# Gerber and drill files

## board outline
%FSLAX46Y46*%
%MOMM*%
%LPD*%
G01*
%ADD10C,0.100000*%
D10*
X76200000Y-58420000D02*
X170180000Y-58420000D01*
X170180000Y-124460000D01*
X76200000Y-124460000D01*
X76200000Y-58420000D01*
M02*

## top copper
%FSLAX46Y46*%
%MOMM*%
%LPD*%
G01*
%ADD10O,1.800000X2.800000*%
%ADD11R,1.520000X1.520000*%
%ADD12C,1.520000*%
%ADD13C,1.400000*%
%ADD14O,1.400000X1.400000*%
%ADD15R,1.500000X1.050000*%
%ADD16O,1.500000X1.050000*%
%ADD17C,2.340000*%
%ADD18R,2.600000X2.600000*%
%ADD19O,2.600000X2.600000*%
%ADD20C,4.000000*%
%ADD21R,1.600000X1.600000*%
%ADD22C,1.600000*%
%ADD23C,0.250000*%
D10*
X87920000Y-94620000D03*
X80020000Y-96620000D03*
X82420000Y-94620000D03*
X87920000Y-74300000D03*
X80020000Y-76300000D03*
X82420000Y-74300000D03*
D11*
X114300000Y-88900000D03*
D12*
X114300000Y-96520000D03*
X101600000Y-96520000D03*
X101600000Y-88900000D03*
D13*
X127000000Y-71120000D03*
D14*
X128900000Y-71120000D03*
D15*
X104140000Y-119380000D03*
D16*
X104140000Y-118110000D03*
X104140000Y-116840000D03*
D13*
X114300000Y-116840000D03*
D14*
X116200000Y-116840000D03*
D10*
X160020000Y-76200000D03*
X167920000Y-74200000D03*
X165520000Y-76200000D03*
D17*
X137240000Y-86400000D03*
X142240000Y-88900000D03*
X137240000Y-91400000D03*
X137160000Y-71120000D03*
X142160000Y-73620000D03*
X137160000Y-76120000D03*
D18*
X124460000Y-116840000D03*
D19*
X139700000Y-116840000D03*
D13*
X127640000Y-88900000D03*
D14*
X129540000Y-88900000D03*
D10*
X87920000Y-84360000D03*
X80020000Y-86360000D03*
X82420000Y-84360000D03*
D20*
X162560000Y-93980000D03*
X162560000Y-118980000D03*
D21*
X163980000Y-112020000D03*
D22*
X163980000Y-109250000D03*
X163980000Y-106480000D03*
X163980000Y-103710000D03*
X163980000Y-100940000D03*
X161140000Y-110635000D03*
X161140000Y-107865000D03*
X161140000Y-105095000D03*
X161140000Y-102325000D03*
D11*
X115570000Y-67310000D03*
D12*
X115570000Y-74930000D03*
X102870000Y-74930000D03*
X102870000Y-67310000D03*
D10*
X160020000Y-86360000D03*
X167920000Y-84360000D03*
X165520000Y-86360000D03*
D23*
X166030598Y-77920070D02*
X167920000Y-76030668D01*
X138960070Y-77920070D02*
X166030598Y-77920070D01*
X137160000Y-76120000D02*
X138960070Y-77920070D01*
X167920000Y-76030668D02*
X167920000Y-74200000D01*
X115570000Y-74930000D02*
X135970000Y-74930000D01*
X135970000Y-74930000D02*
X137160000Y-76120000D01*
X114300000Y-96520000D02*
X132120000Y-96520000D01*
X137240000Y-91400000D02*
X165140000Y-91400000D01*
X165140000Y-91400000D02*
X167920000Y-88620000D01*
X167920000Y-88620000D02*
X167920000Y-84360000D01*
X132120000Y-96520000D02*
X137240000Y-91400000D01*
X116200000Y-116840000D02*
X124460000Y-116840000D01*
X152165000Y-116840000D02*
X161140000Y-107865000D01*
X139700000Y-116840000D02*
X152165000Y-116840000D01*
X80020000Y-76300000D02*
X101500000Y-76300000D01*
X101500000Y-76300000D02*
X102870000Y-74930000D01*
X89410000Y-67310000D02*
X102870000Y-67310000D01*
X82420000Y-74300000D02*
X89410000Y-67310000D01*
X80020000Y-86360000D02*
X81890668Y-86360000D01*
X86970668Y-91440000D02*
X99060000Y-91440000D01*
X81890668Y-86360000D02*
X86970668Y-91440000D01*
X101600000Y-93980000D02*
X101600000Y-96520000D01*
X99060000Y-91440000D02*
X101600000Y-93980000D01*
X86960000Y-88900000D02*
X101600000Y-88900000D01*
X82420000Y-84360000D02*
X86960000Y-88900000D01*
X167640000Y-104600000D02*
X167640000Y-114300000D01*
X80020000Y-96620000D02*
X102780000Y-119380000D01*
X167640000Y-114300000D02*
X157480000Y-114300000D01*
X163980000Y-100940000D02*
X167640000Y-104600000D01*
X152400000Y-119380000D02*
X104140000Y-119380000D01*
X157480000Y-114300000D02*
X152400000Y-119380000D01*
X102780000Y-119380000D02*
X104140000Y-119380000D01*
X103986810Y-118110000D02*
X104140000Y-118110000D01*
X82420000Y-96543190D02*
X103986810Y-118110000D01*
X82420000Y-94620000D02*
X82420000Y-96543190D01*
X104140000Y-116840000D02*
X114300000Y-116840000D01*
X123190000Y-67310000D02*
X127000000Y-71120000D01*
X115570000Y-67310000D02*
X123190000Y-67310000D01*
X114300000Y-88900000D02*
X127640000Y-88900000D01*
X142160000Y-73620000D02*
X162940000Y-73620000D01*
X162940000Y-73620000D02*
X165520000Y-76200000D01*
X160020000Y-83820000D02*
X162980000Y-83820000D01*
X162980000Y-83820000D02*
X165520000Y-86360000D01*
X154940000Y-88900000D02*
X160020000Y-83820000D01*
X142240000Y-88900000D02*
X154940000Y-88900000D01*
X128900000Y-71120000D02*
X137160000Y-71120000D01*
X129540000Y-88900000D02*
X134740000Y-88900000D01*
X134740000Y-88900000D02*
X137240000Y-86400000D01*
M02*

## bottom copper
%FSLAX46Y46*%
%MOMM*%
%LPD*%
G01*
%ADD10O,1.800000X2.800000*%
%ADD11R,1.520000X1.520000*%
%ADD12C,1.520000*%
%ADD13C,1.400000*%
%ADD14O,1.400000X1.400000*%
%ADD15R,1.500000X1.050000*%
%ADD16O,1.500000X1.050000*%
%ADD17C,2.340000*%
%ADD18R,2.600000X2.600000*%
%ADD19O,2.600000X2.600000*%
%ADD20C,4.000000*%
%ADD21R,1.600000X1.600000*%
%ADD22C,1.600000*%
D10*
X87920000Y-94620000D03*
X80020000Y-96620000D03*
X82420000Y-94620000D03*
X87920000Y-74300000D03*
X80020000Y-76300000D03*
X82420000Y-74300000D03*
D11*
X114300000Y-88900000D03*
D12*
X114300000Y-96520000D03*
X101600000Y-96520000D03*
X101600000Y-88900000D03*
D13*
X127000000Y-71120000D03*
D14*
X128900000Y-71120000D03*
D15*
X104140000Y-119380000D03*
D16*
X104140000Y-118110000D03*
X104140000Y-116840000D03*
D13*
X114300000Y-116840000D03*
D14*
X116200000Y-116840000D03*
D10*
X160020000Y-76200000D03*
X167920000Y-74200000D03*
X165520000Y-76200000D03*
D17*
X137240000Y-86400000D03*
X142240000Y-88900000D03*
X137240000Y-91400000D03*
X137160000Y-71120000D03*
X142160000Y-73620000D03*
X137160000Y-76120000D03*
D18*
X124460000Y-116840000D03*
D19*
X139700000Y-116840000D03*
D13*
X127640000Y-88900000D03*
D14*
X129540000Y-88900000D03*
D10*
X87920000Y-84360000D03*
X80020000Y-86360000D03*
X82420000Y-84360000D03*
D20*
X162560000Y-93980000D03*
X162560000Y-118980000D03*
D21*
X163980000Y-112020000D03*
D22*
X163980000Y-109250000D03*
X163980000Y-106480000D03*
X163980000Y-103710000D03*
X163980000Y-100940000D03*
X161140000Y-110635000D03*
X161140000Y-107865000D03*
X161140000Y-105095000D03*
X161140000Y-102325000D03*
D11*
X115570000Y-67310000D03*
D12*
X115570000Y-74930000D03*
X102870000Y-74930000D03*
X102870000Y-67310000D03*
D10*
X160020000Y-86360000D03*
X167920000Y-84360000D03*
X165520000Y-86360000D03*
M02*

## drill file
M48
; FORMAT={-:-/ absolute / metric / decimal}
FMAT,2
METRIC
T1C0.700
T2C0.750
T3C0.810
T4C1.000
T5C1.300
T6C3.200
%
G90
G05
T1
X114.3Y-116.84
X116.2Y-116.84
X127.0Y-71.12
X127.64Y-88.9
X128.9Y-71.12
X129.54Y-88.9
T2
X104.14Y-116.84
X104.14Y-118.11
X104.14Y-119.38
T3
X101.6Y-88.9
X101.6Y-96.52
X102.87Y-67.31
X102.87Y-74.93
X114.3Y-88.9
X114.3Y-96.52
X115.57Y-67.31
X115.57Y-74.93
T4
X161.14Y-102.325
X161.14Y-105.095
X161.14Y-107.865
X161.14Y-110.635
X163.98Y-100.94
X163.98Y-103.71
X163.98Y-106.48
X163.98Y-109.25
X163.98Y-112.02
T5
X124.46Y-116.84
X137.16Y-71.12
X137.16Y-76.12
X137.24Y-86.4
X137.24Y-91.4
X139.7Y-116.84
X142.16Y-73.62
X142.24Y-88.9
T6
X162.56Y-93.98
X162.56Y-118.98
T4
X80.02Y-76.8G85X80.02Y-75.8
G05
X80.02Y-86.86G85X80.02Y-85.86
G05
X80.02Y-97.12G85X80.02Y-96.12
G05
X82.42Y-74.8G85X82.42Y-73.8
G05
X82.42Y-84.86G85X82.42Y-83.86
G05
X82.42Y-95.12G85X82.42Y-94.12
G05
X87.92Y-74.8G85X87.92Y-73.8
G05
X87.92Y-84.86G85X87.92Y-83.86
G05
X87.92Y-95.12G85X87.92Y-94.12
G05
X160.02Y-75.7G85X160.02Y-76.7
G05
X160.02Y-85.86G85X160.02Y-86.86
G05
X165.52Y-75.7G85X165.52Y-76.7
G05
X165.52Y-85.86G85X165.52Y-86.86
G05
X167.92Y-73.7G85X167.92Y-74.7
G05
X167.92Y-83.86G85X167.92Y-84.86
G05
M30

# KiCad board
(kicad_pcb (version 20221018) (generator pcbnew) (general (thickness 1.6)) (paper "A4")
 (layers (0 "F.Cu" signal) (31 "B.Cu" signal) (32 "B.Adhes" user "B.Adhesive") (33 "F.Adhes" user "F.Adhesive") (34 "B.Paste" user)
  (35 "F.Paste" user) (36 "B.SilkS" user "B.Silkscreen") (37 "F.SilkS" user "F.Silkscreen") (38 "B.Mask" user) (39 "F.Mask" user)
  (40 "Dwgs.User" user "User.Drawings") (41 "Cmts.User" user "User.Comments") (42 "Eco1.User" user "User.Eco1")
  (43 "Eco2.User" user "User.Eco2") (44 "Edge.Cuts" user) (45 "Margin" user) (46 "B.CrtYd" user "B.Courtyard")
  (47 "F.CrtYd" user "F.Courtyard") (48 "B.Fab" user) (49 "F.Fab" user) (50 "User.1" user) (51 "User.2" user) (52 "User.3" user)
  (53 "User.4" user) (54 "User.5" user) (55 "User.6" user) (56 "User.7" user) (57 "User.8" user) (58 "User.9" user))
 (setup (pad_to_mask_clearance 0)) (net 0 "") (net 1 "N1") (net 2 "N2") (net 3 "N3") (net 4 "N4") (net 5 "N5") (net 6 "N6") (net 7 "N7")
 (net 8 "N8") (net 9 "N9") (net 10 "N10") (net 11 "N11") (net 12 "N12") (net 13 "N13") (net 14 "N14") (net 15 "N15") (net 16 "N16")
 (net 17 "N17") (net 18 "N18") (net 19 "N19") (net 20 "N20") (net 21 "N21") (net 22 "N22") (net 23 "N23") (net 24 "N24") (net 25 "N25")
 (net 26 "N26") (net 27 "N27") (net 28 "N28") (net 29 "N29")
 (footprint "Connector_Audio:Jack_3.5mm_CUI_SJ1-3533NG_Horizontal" (layer "F.Cu") (at 80.02 96.62 90)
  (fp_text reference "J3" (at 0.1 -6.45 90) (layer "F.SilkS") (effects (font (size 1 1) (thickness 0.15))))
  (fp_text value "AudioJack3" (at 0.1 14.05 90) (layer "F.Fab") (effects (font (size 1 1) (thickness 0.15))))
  (pad "R" thru_hole oval (at 2 7.9 90) (size 2.8 1.8) (drill oval 2 1) (layers "*.Cu" "*.Mask") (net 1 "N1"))
  (pad "S" thru_hole oval (at 0 0 90) (size 2.8 1.8) (drill oval 2 1) (layers "*.Cu" "*.Mask") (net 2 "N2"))
  (pad "T" thru_hole oval (at 2 2.4 90) (size 2.8 1.8) (drill oval 2 1) (layers "*.Cu" "*.Mask") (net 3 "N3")))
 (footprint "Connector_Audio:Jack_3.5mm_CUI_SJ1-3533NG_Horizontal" (layer "F.Cu") (at 80.02 76.3 90)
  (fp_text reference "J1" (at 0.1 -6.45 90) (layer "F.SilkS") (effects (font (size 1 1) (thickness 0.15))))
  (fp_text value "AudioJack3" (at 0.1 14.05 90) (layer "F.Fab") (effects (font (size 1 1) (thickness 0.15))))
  (pad "R" thru_hole oval (at 2 7.9 90) (size 2.8 1.8) (drill oval 2 1) (layers "*.Cu" "*.Mask") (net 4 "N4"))
  (pad "S" thru_hole oval (at 0 0 90) (size 2.8 1.8) (drill oval 2 1) (layers "*.Cu" "*.Mask") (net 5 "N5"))
  (pad "T" thru_hole oval (at 2 2.4 90) (size 2.8 1.8) (drill oval 2 1) (layers "*.Cu" "*.Mask") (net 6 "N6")))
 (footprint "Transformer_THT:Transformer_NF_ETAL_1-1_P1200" (layer "F.Cu") (at 114.3 88.9)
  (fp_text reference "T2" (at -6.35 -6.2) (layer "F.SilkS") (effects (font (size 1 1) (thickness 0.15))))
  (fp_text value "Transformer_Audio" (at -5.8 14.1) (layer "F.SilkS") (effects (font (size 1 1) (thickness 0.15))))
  (pad "1" thru_hole rect (at 0 0) (size 1.52 1.52) (drill 0.81) (layers "*.Cu" "*.Mask") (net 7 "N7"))
  (pad "3" thru_hole circle (at 0 7.62) (size 1.52 1.52) (drill 0.81) (layers "*.Cu" "*.Mask") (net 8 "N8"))
  (pad "4" thru_hole circle (at -12.7 7.62) (size 1.52 1.52) (drill 0.81) (layers "*.Cu" "*.Mask") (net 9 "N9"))
  (pad "6" thru_hole circle (at -12.7 0) (size 1.52 1.52) (drill 0.81) (layers "*.Cu" "*.Mask") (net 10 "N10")))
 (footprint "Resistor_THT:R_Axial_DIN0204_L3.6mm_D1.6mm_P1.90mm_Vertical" (layer "F.Cu") (at 127 71.12)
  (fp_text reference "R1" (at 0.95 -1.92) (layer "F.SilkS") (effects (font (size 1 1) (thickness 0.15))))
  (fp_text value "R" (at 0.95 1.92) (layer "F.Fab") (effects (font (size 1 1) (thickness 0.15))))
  (pad "1" thru_hole circle (at 0 0) (size 1.4 1.4) (drill 0.7) (layers "*.Cu" "*.Mask") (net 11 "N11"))
  (pad "2" thru_hole oval (at 1.9 0) (size 1.4 1.4) (drill 0.7) (layers "*.Cu" "*.Mask") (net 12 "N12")))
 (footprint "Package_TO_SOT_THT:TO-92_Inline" (layer "F.Cu") (at 104.14 119.38 90)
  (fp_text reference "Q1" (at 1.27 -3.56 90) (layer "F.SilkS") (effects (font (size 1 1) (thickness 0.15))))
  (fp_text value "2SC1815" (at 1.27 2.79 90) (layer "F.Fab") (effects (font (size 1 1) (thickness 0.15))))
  (pad "1" thru_hole rect (at 0 0 90) (size 1.05 1.5) (drill 0.75) (layers "*.Cu" "*.Mask") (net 2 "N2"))
  (pad "2" thru_hole oval (at 1.27 0 90) (size 1.05 1.5) (drill 0.75) (layers "*.Cu" "*.Mask") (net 3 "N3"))
  (pad "3" thru_hole oval (at 2.54 0 90) (size 1.05 1.5) (drill 0.75) (layers "*.Cu" "*.Mask") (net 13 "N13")))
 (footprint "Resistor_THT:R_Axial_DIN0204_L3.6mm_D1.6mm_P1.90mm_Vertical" (layer "F.Cu") (at 114.3 116.84)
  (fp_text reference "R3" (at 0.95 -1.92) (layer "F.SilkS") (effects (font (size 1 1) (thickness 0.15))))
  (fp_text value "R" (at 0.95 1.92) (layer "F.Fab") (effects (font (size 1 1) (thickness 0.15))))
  (pad "1" thru_hole circle (at 0 0) (size 1.4 1.4) (drill 0.7) (layers "*.Cu" "*.Mask") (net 13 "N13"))
  (pad "2" thru_hole oval (at 1.9 0) (size 1.4 1.4) (drill 0.7) (layers "*.Cu" "*.Mask") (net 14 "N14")))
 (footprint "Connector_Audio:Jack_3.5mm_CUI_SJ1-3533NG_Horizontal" (layer "F.Cu") (at 167.92 74.2 -90)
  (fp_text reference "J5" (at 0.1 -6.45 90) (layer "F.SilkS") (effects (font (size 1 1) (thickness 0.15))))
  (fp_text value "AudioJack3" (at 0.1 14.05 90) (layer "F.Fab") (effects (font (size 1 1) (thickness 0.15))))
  (pad "R" thru_hole oval (at 2 7.9 270) (size 2.8 1.8) (drill oval 2 1) (layers "*.Cu" "*.Mask") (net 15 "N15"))
  (pad "S" thru_hole oval (at 0 0 270) (size 2.8 1.8) (drill oval 2 1) (layers "*.Cu" "*.Mask") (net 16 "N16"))
  (pad "T" thru_hole oval (at 2 2.4 270) (size 2.8 1.8) (drill oval 2 1) (layers "*.Cu" "*.Mask") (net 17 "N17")))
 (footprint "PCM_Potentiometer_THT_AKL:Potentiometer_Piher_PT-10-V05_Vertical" (layer "F.Cu") (at 137.24 91.4)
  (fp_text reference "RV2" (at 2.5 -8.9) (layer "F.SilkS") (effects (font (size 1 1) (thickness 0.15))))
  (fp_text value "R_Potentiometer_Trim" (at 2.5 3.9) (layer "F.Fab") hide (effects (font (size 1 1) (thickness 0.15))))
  (pad "1" thru_hole circle (at 0 -5) (size 2.34 2.34) (drill 1.3) (layers "*.Cu" "*.Mask") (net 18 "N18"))
  (pad "2" thru_hole circle (at 5 -2.5) (size 2.34 2.34) (drill 1.3) (layers "*.Cu" "*.Mask") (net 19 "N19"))
  (pad "3" thru_hole circle (at 0 0) (size 2.34 2.34) (drill 1.3) (layers "*.Cu" "*.Mask") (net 8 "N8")))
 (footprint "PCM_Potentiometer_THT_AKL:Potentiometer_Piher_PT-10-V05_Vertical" (layer "F.Cu") (at 137.16 76.12)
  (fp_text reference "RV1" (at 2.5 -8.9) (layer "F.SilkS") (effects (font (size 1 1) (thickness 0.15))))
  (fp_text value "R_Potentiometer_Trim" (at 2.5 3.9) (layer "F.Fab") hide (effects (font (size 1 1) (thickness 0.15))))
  (pad "1" thru_hole circle (at 0 -5) (size 2.34 2.34) (drill 1.3) (layers "*.Cu" "*.Mask") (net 12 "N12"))
  (pad "2" thru_hole circle (at 5 -2.5) (size 2.34 2.34) (drill 1.3) (layers "*.Cu" "*.Mask") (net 17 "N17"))
  (pad "3" thru_hole circle (at 0 0) (size 2.34 2.34) (drill 1.3) (layers "*.Cu" "*.Mask") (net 16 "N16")))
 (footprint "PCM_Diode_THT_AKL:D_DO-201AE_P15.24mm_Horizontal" (layer "F.Cu") (at 124.46 116.84)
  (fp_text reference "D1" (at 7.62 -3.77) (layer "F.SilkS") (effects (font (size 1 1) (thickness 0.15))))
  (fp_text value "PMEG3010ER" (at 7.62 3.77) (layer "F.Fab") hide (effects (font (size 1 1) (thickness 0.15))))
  (pad "1" thru_hole rect (at 0 0) (size 2.6 2.6) (drill 1.3) (layers "*.Cu" "*.Mask") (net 14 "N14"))
  (pad "2" thru_hole oval (at 15.24 0) (size 2.6 2.6) (drill 1.3) (layers "*.Cu" "*.Mask") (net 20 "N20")))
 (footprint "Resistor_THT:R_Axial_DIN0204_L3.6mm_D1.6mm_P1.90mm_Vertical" (layer "F.Cu") (at 127.64 88.9)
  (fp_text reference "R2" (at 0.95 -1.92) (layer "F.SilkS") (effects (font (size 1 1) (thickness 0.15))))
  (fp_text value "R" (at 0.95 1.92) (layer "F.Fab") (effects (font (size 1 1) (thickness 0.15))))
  (pad "1" thru_hole circle (at 0 0) (size 1.4 1.4) (drill 0.7) (layers "*.Cu" "*.Mask") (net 7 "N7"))
  (pad "2" thru_hole oval (at 1.9 0) (size 1.4 1.4) (drill 0.7) (layers "*.Cu" "*.Mask") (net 18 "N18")))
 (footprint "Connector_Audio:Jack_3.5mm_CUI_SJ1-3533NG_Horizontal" (layer "F.Cu") (at 80.02 86.36 90)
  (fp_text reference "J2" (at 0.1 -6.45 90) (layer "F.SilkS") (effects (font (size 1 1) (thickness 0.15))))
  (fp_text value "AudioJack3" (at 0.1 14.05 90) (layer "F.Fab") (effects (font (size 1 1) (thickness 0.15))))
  (pad "R" thru_hole oval (at 2 7.9 90) (size 2.8 1.8) (drill oval 2 1) (layers "*.Cu" "*.Mask") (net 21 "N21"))
  (pad "S" thru_hole oval (at 0 0 90) (size 2.8 1.8) (drill oval 2 1) (layers "*.Cu" "*.Mask") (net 9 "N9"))
  (pad "T" thru_hole oval (at 2 2.4 90) (size 2.8 1.8) (drill oval 2 1) (layers "*.Cu" "*.Mask") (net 10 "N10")))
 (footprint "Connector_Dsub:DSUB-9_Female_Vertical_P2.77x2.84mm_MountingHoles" (layer "F.Cu") (at 163.98 112.02 -90)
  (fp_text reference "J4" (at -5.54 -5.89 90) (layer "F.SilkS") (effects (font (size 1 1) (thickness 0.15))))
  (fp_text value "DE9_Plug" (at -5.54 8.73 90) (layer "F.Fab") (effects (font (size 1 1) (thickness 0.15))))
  (pad "0" thru_hole circle (at -18.04 1.42 270) (size 4 4) (drill 3.2) (layers "*.Cu" "*.Mask"))
  (pad "0" thru_hole circle (at 6.96 1.42 270) (size 4 4) (drill 3.2) (layers "*.Cu" "*.Mask"))
  (pad "1" thru_hole rect (at 0 0 270) (size 1.6 1.6) (drill 1) (layers "*.Cu" "*.Mask") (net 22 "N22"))
  (pad "2" thru_hole circle (at -2.77 0 270) (size 1.6 1.6) (drill 1) (layers "*.Cu" "*.Mask") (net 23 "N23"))
  (pad "3" thru_hole circle (at -5.54 0 270) (size 1.6 1.6) (drill 1) (layers "*.Cu" "*.Mask") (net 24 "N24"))
  (pad "4" thru_hole circle (at -8.31 0 270) (size 1.6 1.6) (drill 1) (layers "*.Cu" "*.Mask") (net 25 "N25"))
  (pad "5" thru_hole circle (at -11.08 0 270) (size 1.6 1.6) (drill 1) (layers "*.Cu" "*.Mask") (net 2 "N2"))
  (pad "6" thru_hole circle (at -1.385 2.84 270) (size 1.6 1.6) (drill 1) (layers "*.Cu" "*.Mask") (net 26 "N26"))
  (pad "7" thru_hole circle (at -4.155 2.84 270) (size 1.6 1.6) (drill 1) (layers "*.Cu" "*.Mask") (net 20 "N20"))
  (pad "8" thru_hole circle (at -6.925 2.84 270) (size 1.6 1.6) (drill 1) (layers "*.Cu" "*.Mask") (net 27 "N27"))
  (pad "9" thru_hole circle (at -9.695 2.84 270) (size 1.6 1.6) (drill 1) (layers "*.Cu" "*.Mask") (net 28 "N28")))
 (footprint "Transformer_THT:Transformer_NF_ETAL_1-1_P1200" (layer "F.Cu") (at 115.57 67.31)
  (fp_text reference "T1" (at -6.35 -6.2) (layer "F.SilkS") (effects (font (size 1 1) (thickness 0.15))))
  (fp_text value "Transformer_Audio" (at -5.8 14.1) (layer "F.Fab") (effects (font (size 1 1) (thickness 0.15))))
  (pad "1" thru_hole rect (at 0 0) (size 1.52 1.52) (drill 0.81) (layers "*.Cu" "*.Mask") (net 11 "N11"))
  (pad "3" thru_hole circle (at 0 7.62) (size 1.52 1.52) (drill 0.81) (layers "*.Cu" "*.Mask") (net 16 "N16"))
  (pad "4" thru_hole circle (at -12.7 7.62) (size 1.52 1.52) (drill 0.81) (layers "*.Cu" "*.Mask") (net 5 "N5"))
  (pad "6" thru_hole circle (at -12.7 0) (size 1.52 1.52) (drill 0.81) (layers "*.Cu" "*.Mask") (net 6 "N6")))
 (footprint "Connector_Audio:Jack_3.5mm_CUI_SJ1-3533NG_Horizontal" (layer "F.Cu") (at 167.92 84.36 -90)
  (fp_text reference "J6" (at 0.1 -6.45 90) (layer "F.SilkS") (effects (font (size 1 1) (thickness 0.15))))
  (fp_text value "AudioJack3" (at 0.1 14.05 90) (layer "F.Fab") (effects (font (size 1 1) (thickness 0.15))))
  (pad "R" thru_hole oval (at 2 7.9 270) (size 2.8 1.8) (drill oval 2 1) (layers "*.Cu" "*.Mask") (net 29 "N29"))
  (pad "S" thru_hole oval (at 0 0 270) (size 2.8 1.8) (drill oval 2 1) (layers "*.Cu" "*.Mask") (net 8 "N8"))
  (pad "T" thru_hole oval (at 2 2.4 270) (size 2.8 1.8) (drill oval 2 1) (layers "*.Cu" "*.Mask") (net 19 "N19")))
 (gr_rect (start 76.2 58.42) (end 170.18 124.46) (stroke (width 0.1) (type default)) (fill none) (layer "Edge.Cuts"))
 (segment (start 166.030598 77.92007) (end 167.92 76.030668) (width 0.25) (layer "F.Cu") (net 16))
 (segment (start 138.96007 77.92007) (end 166.030598 77.92007) (width 0.25) (layer "F.Cu") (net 16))
 (segment (start 137.16 76.12) (end 138.96007 77.92007) (width 0.25) (layer "F.Cu") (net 16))
 (segment (start 167.92 76.030668) (end 167.92 74.2) (width 0.25) (layer "F.Cu") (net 16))
 (segment (start 115.57 74.93) (end 135.97 74.93) (width 0.25) (layer "F.Cu") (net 16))
 (segment (start 135.97 74.93) (end 137.16 76.12) (width 0.25) (layer "F.Cu") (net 16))
 (segment (start 114.3 96.52) (end 132.12 96.52) (width 0.25) (layer "F.Cu") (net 8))
 (segment (start 137.24 91.4) (end 165.14 91.4) (width 0.25) (layer "F.Cu") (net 8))
 (segment (start 165.14 91.4) (end 167.92 88.62) (width 0.25) (layer "F.Cu") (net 8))
 (segment (start 167.92 88.62) (end 167.92 84.36) (width 0.25) (layer "F.Cu") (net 8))
 (segment (start 132.12 96.52) (end 137.24 91.4) (width 0.25) (layer "F.Cu") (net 8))
 (segment (start 116.2 116.84) (end 124.46 116.84) (width 0.25) (layer "F.Cu") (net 14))
 (segment (start 152.165 116.84) (end 161.14 107.865) (width 0.25) (layer "F.Cu") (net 20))
 (segment (start 139.7 116.84) (end 152.165 116.84) (width 0.25) (layer "F.Cu") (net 20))
 (segment (start 80.02 76.3) (end 101.5 76.3) (width 0.25) (layer "F.Cu") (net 5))
 (segment (start 101.5 76.3) (end 102.87 74.93) (width 0.25) (layer "F.Cu") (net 5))
 (segment (start 89.41 67.31) (end 102.87 67.31) (width 0.25) (layer "F.Cu") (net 6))
 (segment (start 82.42 74.3) (end 89.41 67.31) (width 0.25) (layer "F.Cu") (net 6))
 (segment (start 80.02 86.36) (end 81.890668 86.36) (width 0.25) (layer "F.Cu") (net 9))
 (segment (start 86.970668 91.44) (end 99.06 91.44) (width 0.25) (layer "F.Cu") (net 9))
 (segment (start 81.890668 86.36) (end 86.970668 91.44) (width 0.25) (layer "F.Cu") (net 9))
 (segment (start 101.6 93.98) (end 101.6 96.52) (width 0.25) (layer "F.Cu") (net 9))
 (segment (start 99.06 91.44) (end 101.6 93.98) (width 0.25) (layer "F.Cu") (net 9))
 (segment (start 86.96 88.9) (end 101.6 88.9) (width 0.25) (layer "F.Cu") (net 10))
 (segment (start 82.42 84.36) (end 86.96 88.9) (width 0.25) (layer "F.Cu") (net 10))
 (segment (start 167.64 104.6) (end 167.64 114.3) (width 0.25) (layer "F.Cu") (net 2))
 (segment (start 80.02 96.62) (end 102.78 119.38) (width 0.25) (layer "F.Cu") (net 2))
 (segment (start 167.64 114.3) (end 157.48 114.3) (width 0.25) (layer "F.Cu") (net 2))
 (segment (start 163.98 100.94) (end 167.64 104.6) (width 0.25) (layer "F.Cu") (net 2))
 (segment (start 152.4 119.38) (end 104.14 119.38) (width 0.25) (layer "F.Cu") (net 2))
 (segment (start 157.48 114.3) (end 152.4 119.38) (width 0.25) (layer "F.Cu") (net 2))
 (segment (start 102.78 119.38) (end 104.14 119.38) (width 0.25) (layer "F.Cu") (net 2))
 (segment (start 103.98681 118.11) (end 104.14 118.11) (width 0.25) (layer "F.Cu") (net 3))
 (segment (start 82.42 96.54319) (end 103.98681 118.11) (width 0.25) (layer "F.Cu") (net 3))
 (segment (start 82.42 94.62) (end 82.42 96.54319) (width 0.25) (layer "F.Cu") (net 3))
 (segment (start 104.14 116.84) (end 114.3 116.84) (width 0.25) (layer "F.Cu") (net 13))
 (segment (start 123.19 67.31) (end 127 71.12) (width 0.25) (layer "F.Cu") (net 11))
 (segment (start 115.57 67.31) (end 123.19 67.31) (width 0.25) (layer "F.Cu") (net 11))
 (segment (start 114.3 88.9) (end 127.64 88.9) (width 0.25) (layer "F.Cu") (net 7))
 (segment (start 142.16 73.62) (end 162.94 73.62) (width 0.25) (layer "F.Cu") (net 17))
 (segment (start 162.94 73.62) (end 165.52 76.2) (width 0.25) (layer "F.Cu") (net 17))
 (segment (start 160.02 83.82) (end 162.98 83.82) (width 0.25) (layer "F.Cu") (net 19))
 (segment (start 162.98 83.82) (end 165.52 86.36) (width 0.25) (layer "F.Cu") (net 19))
 (segment (start 154.94 88.9) (end 160.02 83.82) (width 0.25) (layer "F.Cu") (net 19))
 (segment (start 142.24 88.9) (end 154.94 88.9) (width 0.25) (layer "F.Cu") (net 19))
 (segment (start 128.9 71.12) (end 137.16 71.12) (width 0.25) (layer "F.Cu") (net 12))
 (segment (start 129.54 88.9) (end 134.74 88.9) (width 0.25) (layer "F.Cu") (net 18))
 (segment (start 134.74 88.9) (end 137.24 86.4) (width 0.25) (layer "F.Cu") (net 18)))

